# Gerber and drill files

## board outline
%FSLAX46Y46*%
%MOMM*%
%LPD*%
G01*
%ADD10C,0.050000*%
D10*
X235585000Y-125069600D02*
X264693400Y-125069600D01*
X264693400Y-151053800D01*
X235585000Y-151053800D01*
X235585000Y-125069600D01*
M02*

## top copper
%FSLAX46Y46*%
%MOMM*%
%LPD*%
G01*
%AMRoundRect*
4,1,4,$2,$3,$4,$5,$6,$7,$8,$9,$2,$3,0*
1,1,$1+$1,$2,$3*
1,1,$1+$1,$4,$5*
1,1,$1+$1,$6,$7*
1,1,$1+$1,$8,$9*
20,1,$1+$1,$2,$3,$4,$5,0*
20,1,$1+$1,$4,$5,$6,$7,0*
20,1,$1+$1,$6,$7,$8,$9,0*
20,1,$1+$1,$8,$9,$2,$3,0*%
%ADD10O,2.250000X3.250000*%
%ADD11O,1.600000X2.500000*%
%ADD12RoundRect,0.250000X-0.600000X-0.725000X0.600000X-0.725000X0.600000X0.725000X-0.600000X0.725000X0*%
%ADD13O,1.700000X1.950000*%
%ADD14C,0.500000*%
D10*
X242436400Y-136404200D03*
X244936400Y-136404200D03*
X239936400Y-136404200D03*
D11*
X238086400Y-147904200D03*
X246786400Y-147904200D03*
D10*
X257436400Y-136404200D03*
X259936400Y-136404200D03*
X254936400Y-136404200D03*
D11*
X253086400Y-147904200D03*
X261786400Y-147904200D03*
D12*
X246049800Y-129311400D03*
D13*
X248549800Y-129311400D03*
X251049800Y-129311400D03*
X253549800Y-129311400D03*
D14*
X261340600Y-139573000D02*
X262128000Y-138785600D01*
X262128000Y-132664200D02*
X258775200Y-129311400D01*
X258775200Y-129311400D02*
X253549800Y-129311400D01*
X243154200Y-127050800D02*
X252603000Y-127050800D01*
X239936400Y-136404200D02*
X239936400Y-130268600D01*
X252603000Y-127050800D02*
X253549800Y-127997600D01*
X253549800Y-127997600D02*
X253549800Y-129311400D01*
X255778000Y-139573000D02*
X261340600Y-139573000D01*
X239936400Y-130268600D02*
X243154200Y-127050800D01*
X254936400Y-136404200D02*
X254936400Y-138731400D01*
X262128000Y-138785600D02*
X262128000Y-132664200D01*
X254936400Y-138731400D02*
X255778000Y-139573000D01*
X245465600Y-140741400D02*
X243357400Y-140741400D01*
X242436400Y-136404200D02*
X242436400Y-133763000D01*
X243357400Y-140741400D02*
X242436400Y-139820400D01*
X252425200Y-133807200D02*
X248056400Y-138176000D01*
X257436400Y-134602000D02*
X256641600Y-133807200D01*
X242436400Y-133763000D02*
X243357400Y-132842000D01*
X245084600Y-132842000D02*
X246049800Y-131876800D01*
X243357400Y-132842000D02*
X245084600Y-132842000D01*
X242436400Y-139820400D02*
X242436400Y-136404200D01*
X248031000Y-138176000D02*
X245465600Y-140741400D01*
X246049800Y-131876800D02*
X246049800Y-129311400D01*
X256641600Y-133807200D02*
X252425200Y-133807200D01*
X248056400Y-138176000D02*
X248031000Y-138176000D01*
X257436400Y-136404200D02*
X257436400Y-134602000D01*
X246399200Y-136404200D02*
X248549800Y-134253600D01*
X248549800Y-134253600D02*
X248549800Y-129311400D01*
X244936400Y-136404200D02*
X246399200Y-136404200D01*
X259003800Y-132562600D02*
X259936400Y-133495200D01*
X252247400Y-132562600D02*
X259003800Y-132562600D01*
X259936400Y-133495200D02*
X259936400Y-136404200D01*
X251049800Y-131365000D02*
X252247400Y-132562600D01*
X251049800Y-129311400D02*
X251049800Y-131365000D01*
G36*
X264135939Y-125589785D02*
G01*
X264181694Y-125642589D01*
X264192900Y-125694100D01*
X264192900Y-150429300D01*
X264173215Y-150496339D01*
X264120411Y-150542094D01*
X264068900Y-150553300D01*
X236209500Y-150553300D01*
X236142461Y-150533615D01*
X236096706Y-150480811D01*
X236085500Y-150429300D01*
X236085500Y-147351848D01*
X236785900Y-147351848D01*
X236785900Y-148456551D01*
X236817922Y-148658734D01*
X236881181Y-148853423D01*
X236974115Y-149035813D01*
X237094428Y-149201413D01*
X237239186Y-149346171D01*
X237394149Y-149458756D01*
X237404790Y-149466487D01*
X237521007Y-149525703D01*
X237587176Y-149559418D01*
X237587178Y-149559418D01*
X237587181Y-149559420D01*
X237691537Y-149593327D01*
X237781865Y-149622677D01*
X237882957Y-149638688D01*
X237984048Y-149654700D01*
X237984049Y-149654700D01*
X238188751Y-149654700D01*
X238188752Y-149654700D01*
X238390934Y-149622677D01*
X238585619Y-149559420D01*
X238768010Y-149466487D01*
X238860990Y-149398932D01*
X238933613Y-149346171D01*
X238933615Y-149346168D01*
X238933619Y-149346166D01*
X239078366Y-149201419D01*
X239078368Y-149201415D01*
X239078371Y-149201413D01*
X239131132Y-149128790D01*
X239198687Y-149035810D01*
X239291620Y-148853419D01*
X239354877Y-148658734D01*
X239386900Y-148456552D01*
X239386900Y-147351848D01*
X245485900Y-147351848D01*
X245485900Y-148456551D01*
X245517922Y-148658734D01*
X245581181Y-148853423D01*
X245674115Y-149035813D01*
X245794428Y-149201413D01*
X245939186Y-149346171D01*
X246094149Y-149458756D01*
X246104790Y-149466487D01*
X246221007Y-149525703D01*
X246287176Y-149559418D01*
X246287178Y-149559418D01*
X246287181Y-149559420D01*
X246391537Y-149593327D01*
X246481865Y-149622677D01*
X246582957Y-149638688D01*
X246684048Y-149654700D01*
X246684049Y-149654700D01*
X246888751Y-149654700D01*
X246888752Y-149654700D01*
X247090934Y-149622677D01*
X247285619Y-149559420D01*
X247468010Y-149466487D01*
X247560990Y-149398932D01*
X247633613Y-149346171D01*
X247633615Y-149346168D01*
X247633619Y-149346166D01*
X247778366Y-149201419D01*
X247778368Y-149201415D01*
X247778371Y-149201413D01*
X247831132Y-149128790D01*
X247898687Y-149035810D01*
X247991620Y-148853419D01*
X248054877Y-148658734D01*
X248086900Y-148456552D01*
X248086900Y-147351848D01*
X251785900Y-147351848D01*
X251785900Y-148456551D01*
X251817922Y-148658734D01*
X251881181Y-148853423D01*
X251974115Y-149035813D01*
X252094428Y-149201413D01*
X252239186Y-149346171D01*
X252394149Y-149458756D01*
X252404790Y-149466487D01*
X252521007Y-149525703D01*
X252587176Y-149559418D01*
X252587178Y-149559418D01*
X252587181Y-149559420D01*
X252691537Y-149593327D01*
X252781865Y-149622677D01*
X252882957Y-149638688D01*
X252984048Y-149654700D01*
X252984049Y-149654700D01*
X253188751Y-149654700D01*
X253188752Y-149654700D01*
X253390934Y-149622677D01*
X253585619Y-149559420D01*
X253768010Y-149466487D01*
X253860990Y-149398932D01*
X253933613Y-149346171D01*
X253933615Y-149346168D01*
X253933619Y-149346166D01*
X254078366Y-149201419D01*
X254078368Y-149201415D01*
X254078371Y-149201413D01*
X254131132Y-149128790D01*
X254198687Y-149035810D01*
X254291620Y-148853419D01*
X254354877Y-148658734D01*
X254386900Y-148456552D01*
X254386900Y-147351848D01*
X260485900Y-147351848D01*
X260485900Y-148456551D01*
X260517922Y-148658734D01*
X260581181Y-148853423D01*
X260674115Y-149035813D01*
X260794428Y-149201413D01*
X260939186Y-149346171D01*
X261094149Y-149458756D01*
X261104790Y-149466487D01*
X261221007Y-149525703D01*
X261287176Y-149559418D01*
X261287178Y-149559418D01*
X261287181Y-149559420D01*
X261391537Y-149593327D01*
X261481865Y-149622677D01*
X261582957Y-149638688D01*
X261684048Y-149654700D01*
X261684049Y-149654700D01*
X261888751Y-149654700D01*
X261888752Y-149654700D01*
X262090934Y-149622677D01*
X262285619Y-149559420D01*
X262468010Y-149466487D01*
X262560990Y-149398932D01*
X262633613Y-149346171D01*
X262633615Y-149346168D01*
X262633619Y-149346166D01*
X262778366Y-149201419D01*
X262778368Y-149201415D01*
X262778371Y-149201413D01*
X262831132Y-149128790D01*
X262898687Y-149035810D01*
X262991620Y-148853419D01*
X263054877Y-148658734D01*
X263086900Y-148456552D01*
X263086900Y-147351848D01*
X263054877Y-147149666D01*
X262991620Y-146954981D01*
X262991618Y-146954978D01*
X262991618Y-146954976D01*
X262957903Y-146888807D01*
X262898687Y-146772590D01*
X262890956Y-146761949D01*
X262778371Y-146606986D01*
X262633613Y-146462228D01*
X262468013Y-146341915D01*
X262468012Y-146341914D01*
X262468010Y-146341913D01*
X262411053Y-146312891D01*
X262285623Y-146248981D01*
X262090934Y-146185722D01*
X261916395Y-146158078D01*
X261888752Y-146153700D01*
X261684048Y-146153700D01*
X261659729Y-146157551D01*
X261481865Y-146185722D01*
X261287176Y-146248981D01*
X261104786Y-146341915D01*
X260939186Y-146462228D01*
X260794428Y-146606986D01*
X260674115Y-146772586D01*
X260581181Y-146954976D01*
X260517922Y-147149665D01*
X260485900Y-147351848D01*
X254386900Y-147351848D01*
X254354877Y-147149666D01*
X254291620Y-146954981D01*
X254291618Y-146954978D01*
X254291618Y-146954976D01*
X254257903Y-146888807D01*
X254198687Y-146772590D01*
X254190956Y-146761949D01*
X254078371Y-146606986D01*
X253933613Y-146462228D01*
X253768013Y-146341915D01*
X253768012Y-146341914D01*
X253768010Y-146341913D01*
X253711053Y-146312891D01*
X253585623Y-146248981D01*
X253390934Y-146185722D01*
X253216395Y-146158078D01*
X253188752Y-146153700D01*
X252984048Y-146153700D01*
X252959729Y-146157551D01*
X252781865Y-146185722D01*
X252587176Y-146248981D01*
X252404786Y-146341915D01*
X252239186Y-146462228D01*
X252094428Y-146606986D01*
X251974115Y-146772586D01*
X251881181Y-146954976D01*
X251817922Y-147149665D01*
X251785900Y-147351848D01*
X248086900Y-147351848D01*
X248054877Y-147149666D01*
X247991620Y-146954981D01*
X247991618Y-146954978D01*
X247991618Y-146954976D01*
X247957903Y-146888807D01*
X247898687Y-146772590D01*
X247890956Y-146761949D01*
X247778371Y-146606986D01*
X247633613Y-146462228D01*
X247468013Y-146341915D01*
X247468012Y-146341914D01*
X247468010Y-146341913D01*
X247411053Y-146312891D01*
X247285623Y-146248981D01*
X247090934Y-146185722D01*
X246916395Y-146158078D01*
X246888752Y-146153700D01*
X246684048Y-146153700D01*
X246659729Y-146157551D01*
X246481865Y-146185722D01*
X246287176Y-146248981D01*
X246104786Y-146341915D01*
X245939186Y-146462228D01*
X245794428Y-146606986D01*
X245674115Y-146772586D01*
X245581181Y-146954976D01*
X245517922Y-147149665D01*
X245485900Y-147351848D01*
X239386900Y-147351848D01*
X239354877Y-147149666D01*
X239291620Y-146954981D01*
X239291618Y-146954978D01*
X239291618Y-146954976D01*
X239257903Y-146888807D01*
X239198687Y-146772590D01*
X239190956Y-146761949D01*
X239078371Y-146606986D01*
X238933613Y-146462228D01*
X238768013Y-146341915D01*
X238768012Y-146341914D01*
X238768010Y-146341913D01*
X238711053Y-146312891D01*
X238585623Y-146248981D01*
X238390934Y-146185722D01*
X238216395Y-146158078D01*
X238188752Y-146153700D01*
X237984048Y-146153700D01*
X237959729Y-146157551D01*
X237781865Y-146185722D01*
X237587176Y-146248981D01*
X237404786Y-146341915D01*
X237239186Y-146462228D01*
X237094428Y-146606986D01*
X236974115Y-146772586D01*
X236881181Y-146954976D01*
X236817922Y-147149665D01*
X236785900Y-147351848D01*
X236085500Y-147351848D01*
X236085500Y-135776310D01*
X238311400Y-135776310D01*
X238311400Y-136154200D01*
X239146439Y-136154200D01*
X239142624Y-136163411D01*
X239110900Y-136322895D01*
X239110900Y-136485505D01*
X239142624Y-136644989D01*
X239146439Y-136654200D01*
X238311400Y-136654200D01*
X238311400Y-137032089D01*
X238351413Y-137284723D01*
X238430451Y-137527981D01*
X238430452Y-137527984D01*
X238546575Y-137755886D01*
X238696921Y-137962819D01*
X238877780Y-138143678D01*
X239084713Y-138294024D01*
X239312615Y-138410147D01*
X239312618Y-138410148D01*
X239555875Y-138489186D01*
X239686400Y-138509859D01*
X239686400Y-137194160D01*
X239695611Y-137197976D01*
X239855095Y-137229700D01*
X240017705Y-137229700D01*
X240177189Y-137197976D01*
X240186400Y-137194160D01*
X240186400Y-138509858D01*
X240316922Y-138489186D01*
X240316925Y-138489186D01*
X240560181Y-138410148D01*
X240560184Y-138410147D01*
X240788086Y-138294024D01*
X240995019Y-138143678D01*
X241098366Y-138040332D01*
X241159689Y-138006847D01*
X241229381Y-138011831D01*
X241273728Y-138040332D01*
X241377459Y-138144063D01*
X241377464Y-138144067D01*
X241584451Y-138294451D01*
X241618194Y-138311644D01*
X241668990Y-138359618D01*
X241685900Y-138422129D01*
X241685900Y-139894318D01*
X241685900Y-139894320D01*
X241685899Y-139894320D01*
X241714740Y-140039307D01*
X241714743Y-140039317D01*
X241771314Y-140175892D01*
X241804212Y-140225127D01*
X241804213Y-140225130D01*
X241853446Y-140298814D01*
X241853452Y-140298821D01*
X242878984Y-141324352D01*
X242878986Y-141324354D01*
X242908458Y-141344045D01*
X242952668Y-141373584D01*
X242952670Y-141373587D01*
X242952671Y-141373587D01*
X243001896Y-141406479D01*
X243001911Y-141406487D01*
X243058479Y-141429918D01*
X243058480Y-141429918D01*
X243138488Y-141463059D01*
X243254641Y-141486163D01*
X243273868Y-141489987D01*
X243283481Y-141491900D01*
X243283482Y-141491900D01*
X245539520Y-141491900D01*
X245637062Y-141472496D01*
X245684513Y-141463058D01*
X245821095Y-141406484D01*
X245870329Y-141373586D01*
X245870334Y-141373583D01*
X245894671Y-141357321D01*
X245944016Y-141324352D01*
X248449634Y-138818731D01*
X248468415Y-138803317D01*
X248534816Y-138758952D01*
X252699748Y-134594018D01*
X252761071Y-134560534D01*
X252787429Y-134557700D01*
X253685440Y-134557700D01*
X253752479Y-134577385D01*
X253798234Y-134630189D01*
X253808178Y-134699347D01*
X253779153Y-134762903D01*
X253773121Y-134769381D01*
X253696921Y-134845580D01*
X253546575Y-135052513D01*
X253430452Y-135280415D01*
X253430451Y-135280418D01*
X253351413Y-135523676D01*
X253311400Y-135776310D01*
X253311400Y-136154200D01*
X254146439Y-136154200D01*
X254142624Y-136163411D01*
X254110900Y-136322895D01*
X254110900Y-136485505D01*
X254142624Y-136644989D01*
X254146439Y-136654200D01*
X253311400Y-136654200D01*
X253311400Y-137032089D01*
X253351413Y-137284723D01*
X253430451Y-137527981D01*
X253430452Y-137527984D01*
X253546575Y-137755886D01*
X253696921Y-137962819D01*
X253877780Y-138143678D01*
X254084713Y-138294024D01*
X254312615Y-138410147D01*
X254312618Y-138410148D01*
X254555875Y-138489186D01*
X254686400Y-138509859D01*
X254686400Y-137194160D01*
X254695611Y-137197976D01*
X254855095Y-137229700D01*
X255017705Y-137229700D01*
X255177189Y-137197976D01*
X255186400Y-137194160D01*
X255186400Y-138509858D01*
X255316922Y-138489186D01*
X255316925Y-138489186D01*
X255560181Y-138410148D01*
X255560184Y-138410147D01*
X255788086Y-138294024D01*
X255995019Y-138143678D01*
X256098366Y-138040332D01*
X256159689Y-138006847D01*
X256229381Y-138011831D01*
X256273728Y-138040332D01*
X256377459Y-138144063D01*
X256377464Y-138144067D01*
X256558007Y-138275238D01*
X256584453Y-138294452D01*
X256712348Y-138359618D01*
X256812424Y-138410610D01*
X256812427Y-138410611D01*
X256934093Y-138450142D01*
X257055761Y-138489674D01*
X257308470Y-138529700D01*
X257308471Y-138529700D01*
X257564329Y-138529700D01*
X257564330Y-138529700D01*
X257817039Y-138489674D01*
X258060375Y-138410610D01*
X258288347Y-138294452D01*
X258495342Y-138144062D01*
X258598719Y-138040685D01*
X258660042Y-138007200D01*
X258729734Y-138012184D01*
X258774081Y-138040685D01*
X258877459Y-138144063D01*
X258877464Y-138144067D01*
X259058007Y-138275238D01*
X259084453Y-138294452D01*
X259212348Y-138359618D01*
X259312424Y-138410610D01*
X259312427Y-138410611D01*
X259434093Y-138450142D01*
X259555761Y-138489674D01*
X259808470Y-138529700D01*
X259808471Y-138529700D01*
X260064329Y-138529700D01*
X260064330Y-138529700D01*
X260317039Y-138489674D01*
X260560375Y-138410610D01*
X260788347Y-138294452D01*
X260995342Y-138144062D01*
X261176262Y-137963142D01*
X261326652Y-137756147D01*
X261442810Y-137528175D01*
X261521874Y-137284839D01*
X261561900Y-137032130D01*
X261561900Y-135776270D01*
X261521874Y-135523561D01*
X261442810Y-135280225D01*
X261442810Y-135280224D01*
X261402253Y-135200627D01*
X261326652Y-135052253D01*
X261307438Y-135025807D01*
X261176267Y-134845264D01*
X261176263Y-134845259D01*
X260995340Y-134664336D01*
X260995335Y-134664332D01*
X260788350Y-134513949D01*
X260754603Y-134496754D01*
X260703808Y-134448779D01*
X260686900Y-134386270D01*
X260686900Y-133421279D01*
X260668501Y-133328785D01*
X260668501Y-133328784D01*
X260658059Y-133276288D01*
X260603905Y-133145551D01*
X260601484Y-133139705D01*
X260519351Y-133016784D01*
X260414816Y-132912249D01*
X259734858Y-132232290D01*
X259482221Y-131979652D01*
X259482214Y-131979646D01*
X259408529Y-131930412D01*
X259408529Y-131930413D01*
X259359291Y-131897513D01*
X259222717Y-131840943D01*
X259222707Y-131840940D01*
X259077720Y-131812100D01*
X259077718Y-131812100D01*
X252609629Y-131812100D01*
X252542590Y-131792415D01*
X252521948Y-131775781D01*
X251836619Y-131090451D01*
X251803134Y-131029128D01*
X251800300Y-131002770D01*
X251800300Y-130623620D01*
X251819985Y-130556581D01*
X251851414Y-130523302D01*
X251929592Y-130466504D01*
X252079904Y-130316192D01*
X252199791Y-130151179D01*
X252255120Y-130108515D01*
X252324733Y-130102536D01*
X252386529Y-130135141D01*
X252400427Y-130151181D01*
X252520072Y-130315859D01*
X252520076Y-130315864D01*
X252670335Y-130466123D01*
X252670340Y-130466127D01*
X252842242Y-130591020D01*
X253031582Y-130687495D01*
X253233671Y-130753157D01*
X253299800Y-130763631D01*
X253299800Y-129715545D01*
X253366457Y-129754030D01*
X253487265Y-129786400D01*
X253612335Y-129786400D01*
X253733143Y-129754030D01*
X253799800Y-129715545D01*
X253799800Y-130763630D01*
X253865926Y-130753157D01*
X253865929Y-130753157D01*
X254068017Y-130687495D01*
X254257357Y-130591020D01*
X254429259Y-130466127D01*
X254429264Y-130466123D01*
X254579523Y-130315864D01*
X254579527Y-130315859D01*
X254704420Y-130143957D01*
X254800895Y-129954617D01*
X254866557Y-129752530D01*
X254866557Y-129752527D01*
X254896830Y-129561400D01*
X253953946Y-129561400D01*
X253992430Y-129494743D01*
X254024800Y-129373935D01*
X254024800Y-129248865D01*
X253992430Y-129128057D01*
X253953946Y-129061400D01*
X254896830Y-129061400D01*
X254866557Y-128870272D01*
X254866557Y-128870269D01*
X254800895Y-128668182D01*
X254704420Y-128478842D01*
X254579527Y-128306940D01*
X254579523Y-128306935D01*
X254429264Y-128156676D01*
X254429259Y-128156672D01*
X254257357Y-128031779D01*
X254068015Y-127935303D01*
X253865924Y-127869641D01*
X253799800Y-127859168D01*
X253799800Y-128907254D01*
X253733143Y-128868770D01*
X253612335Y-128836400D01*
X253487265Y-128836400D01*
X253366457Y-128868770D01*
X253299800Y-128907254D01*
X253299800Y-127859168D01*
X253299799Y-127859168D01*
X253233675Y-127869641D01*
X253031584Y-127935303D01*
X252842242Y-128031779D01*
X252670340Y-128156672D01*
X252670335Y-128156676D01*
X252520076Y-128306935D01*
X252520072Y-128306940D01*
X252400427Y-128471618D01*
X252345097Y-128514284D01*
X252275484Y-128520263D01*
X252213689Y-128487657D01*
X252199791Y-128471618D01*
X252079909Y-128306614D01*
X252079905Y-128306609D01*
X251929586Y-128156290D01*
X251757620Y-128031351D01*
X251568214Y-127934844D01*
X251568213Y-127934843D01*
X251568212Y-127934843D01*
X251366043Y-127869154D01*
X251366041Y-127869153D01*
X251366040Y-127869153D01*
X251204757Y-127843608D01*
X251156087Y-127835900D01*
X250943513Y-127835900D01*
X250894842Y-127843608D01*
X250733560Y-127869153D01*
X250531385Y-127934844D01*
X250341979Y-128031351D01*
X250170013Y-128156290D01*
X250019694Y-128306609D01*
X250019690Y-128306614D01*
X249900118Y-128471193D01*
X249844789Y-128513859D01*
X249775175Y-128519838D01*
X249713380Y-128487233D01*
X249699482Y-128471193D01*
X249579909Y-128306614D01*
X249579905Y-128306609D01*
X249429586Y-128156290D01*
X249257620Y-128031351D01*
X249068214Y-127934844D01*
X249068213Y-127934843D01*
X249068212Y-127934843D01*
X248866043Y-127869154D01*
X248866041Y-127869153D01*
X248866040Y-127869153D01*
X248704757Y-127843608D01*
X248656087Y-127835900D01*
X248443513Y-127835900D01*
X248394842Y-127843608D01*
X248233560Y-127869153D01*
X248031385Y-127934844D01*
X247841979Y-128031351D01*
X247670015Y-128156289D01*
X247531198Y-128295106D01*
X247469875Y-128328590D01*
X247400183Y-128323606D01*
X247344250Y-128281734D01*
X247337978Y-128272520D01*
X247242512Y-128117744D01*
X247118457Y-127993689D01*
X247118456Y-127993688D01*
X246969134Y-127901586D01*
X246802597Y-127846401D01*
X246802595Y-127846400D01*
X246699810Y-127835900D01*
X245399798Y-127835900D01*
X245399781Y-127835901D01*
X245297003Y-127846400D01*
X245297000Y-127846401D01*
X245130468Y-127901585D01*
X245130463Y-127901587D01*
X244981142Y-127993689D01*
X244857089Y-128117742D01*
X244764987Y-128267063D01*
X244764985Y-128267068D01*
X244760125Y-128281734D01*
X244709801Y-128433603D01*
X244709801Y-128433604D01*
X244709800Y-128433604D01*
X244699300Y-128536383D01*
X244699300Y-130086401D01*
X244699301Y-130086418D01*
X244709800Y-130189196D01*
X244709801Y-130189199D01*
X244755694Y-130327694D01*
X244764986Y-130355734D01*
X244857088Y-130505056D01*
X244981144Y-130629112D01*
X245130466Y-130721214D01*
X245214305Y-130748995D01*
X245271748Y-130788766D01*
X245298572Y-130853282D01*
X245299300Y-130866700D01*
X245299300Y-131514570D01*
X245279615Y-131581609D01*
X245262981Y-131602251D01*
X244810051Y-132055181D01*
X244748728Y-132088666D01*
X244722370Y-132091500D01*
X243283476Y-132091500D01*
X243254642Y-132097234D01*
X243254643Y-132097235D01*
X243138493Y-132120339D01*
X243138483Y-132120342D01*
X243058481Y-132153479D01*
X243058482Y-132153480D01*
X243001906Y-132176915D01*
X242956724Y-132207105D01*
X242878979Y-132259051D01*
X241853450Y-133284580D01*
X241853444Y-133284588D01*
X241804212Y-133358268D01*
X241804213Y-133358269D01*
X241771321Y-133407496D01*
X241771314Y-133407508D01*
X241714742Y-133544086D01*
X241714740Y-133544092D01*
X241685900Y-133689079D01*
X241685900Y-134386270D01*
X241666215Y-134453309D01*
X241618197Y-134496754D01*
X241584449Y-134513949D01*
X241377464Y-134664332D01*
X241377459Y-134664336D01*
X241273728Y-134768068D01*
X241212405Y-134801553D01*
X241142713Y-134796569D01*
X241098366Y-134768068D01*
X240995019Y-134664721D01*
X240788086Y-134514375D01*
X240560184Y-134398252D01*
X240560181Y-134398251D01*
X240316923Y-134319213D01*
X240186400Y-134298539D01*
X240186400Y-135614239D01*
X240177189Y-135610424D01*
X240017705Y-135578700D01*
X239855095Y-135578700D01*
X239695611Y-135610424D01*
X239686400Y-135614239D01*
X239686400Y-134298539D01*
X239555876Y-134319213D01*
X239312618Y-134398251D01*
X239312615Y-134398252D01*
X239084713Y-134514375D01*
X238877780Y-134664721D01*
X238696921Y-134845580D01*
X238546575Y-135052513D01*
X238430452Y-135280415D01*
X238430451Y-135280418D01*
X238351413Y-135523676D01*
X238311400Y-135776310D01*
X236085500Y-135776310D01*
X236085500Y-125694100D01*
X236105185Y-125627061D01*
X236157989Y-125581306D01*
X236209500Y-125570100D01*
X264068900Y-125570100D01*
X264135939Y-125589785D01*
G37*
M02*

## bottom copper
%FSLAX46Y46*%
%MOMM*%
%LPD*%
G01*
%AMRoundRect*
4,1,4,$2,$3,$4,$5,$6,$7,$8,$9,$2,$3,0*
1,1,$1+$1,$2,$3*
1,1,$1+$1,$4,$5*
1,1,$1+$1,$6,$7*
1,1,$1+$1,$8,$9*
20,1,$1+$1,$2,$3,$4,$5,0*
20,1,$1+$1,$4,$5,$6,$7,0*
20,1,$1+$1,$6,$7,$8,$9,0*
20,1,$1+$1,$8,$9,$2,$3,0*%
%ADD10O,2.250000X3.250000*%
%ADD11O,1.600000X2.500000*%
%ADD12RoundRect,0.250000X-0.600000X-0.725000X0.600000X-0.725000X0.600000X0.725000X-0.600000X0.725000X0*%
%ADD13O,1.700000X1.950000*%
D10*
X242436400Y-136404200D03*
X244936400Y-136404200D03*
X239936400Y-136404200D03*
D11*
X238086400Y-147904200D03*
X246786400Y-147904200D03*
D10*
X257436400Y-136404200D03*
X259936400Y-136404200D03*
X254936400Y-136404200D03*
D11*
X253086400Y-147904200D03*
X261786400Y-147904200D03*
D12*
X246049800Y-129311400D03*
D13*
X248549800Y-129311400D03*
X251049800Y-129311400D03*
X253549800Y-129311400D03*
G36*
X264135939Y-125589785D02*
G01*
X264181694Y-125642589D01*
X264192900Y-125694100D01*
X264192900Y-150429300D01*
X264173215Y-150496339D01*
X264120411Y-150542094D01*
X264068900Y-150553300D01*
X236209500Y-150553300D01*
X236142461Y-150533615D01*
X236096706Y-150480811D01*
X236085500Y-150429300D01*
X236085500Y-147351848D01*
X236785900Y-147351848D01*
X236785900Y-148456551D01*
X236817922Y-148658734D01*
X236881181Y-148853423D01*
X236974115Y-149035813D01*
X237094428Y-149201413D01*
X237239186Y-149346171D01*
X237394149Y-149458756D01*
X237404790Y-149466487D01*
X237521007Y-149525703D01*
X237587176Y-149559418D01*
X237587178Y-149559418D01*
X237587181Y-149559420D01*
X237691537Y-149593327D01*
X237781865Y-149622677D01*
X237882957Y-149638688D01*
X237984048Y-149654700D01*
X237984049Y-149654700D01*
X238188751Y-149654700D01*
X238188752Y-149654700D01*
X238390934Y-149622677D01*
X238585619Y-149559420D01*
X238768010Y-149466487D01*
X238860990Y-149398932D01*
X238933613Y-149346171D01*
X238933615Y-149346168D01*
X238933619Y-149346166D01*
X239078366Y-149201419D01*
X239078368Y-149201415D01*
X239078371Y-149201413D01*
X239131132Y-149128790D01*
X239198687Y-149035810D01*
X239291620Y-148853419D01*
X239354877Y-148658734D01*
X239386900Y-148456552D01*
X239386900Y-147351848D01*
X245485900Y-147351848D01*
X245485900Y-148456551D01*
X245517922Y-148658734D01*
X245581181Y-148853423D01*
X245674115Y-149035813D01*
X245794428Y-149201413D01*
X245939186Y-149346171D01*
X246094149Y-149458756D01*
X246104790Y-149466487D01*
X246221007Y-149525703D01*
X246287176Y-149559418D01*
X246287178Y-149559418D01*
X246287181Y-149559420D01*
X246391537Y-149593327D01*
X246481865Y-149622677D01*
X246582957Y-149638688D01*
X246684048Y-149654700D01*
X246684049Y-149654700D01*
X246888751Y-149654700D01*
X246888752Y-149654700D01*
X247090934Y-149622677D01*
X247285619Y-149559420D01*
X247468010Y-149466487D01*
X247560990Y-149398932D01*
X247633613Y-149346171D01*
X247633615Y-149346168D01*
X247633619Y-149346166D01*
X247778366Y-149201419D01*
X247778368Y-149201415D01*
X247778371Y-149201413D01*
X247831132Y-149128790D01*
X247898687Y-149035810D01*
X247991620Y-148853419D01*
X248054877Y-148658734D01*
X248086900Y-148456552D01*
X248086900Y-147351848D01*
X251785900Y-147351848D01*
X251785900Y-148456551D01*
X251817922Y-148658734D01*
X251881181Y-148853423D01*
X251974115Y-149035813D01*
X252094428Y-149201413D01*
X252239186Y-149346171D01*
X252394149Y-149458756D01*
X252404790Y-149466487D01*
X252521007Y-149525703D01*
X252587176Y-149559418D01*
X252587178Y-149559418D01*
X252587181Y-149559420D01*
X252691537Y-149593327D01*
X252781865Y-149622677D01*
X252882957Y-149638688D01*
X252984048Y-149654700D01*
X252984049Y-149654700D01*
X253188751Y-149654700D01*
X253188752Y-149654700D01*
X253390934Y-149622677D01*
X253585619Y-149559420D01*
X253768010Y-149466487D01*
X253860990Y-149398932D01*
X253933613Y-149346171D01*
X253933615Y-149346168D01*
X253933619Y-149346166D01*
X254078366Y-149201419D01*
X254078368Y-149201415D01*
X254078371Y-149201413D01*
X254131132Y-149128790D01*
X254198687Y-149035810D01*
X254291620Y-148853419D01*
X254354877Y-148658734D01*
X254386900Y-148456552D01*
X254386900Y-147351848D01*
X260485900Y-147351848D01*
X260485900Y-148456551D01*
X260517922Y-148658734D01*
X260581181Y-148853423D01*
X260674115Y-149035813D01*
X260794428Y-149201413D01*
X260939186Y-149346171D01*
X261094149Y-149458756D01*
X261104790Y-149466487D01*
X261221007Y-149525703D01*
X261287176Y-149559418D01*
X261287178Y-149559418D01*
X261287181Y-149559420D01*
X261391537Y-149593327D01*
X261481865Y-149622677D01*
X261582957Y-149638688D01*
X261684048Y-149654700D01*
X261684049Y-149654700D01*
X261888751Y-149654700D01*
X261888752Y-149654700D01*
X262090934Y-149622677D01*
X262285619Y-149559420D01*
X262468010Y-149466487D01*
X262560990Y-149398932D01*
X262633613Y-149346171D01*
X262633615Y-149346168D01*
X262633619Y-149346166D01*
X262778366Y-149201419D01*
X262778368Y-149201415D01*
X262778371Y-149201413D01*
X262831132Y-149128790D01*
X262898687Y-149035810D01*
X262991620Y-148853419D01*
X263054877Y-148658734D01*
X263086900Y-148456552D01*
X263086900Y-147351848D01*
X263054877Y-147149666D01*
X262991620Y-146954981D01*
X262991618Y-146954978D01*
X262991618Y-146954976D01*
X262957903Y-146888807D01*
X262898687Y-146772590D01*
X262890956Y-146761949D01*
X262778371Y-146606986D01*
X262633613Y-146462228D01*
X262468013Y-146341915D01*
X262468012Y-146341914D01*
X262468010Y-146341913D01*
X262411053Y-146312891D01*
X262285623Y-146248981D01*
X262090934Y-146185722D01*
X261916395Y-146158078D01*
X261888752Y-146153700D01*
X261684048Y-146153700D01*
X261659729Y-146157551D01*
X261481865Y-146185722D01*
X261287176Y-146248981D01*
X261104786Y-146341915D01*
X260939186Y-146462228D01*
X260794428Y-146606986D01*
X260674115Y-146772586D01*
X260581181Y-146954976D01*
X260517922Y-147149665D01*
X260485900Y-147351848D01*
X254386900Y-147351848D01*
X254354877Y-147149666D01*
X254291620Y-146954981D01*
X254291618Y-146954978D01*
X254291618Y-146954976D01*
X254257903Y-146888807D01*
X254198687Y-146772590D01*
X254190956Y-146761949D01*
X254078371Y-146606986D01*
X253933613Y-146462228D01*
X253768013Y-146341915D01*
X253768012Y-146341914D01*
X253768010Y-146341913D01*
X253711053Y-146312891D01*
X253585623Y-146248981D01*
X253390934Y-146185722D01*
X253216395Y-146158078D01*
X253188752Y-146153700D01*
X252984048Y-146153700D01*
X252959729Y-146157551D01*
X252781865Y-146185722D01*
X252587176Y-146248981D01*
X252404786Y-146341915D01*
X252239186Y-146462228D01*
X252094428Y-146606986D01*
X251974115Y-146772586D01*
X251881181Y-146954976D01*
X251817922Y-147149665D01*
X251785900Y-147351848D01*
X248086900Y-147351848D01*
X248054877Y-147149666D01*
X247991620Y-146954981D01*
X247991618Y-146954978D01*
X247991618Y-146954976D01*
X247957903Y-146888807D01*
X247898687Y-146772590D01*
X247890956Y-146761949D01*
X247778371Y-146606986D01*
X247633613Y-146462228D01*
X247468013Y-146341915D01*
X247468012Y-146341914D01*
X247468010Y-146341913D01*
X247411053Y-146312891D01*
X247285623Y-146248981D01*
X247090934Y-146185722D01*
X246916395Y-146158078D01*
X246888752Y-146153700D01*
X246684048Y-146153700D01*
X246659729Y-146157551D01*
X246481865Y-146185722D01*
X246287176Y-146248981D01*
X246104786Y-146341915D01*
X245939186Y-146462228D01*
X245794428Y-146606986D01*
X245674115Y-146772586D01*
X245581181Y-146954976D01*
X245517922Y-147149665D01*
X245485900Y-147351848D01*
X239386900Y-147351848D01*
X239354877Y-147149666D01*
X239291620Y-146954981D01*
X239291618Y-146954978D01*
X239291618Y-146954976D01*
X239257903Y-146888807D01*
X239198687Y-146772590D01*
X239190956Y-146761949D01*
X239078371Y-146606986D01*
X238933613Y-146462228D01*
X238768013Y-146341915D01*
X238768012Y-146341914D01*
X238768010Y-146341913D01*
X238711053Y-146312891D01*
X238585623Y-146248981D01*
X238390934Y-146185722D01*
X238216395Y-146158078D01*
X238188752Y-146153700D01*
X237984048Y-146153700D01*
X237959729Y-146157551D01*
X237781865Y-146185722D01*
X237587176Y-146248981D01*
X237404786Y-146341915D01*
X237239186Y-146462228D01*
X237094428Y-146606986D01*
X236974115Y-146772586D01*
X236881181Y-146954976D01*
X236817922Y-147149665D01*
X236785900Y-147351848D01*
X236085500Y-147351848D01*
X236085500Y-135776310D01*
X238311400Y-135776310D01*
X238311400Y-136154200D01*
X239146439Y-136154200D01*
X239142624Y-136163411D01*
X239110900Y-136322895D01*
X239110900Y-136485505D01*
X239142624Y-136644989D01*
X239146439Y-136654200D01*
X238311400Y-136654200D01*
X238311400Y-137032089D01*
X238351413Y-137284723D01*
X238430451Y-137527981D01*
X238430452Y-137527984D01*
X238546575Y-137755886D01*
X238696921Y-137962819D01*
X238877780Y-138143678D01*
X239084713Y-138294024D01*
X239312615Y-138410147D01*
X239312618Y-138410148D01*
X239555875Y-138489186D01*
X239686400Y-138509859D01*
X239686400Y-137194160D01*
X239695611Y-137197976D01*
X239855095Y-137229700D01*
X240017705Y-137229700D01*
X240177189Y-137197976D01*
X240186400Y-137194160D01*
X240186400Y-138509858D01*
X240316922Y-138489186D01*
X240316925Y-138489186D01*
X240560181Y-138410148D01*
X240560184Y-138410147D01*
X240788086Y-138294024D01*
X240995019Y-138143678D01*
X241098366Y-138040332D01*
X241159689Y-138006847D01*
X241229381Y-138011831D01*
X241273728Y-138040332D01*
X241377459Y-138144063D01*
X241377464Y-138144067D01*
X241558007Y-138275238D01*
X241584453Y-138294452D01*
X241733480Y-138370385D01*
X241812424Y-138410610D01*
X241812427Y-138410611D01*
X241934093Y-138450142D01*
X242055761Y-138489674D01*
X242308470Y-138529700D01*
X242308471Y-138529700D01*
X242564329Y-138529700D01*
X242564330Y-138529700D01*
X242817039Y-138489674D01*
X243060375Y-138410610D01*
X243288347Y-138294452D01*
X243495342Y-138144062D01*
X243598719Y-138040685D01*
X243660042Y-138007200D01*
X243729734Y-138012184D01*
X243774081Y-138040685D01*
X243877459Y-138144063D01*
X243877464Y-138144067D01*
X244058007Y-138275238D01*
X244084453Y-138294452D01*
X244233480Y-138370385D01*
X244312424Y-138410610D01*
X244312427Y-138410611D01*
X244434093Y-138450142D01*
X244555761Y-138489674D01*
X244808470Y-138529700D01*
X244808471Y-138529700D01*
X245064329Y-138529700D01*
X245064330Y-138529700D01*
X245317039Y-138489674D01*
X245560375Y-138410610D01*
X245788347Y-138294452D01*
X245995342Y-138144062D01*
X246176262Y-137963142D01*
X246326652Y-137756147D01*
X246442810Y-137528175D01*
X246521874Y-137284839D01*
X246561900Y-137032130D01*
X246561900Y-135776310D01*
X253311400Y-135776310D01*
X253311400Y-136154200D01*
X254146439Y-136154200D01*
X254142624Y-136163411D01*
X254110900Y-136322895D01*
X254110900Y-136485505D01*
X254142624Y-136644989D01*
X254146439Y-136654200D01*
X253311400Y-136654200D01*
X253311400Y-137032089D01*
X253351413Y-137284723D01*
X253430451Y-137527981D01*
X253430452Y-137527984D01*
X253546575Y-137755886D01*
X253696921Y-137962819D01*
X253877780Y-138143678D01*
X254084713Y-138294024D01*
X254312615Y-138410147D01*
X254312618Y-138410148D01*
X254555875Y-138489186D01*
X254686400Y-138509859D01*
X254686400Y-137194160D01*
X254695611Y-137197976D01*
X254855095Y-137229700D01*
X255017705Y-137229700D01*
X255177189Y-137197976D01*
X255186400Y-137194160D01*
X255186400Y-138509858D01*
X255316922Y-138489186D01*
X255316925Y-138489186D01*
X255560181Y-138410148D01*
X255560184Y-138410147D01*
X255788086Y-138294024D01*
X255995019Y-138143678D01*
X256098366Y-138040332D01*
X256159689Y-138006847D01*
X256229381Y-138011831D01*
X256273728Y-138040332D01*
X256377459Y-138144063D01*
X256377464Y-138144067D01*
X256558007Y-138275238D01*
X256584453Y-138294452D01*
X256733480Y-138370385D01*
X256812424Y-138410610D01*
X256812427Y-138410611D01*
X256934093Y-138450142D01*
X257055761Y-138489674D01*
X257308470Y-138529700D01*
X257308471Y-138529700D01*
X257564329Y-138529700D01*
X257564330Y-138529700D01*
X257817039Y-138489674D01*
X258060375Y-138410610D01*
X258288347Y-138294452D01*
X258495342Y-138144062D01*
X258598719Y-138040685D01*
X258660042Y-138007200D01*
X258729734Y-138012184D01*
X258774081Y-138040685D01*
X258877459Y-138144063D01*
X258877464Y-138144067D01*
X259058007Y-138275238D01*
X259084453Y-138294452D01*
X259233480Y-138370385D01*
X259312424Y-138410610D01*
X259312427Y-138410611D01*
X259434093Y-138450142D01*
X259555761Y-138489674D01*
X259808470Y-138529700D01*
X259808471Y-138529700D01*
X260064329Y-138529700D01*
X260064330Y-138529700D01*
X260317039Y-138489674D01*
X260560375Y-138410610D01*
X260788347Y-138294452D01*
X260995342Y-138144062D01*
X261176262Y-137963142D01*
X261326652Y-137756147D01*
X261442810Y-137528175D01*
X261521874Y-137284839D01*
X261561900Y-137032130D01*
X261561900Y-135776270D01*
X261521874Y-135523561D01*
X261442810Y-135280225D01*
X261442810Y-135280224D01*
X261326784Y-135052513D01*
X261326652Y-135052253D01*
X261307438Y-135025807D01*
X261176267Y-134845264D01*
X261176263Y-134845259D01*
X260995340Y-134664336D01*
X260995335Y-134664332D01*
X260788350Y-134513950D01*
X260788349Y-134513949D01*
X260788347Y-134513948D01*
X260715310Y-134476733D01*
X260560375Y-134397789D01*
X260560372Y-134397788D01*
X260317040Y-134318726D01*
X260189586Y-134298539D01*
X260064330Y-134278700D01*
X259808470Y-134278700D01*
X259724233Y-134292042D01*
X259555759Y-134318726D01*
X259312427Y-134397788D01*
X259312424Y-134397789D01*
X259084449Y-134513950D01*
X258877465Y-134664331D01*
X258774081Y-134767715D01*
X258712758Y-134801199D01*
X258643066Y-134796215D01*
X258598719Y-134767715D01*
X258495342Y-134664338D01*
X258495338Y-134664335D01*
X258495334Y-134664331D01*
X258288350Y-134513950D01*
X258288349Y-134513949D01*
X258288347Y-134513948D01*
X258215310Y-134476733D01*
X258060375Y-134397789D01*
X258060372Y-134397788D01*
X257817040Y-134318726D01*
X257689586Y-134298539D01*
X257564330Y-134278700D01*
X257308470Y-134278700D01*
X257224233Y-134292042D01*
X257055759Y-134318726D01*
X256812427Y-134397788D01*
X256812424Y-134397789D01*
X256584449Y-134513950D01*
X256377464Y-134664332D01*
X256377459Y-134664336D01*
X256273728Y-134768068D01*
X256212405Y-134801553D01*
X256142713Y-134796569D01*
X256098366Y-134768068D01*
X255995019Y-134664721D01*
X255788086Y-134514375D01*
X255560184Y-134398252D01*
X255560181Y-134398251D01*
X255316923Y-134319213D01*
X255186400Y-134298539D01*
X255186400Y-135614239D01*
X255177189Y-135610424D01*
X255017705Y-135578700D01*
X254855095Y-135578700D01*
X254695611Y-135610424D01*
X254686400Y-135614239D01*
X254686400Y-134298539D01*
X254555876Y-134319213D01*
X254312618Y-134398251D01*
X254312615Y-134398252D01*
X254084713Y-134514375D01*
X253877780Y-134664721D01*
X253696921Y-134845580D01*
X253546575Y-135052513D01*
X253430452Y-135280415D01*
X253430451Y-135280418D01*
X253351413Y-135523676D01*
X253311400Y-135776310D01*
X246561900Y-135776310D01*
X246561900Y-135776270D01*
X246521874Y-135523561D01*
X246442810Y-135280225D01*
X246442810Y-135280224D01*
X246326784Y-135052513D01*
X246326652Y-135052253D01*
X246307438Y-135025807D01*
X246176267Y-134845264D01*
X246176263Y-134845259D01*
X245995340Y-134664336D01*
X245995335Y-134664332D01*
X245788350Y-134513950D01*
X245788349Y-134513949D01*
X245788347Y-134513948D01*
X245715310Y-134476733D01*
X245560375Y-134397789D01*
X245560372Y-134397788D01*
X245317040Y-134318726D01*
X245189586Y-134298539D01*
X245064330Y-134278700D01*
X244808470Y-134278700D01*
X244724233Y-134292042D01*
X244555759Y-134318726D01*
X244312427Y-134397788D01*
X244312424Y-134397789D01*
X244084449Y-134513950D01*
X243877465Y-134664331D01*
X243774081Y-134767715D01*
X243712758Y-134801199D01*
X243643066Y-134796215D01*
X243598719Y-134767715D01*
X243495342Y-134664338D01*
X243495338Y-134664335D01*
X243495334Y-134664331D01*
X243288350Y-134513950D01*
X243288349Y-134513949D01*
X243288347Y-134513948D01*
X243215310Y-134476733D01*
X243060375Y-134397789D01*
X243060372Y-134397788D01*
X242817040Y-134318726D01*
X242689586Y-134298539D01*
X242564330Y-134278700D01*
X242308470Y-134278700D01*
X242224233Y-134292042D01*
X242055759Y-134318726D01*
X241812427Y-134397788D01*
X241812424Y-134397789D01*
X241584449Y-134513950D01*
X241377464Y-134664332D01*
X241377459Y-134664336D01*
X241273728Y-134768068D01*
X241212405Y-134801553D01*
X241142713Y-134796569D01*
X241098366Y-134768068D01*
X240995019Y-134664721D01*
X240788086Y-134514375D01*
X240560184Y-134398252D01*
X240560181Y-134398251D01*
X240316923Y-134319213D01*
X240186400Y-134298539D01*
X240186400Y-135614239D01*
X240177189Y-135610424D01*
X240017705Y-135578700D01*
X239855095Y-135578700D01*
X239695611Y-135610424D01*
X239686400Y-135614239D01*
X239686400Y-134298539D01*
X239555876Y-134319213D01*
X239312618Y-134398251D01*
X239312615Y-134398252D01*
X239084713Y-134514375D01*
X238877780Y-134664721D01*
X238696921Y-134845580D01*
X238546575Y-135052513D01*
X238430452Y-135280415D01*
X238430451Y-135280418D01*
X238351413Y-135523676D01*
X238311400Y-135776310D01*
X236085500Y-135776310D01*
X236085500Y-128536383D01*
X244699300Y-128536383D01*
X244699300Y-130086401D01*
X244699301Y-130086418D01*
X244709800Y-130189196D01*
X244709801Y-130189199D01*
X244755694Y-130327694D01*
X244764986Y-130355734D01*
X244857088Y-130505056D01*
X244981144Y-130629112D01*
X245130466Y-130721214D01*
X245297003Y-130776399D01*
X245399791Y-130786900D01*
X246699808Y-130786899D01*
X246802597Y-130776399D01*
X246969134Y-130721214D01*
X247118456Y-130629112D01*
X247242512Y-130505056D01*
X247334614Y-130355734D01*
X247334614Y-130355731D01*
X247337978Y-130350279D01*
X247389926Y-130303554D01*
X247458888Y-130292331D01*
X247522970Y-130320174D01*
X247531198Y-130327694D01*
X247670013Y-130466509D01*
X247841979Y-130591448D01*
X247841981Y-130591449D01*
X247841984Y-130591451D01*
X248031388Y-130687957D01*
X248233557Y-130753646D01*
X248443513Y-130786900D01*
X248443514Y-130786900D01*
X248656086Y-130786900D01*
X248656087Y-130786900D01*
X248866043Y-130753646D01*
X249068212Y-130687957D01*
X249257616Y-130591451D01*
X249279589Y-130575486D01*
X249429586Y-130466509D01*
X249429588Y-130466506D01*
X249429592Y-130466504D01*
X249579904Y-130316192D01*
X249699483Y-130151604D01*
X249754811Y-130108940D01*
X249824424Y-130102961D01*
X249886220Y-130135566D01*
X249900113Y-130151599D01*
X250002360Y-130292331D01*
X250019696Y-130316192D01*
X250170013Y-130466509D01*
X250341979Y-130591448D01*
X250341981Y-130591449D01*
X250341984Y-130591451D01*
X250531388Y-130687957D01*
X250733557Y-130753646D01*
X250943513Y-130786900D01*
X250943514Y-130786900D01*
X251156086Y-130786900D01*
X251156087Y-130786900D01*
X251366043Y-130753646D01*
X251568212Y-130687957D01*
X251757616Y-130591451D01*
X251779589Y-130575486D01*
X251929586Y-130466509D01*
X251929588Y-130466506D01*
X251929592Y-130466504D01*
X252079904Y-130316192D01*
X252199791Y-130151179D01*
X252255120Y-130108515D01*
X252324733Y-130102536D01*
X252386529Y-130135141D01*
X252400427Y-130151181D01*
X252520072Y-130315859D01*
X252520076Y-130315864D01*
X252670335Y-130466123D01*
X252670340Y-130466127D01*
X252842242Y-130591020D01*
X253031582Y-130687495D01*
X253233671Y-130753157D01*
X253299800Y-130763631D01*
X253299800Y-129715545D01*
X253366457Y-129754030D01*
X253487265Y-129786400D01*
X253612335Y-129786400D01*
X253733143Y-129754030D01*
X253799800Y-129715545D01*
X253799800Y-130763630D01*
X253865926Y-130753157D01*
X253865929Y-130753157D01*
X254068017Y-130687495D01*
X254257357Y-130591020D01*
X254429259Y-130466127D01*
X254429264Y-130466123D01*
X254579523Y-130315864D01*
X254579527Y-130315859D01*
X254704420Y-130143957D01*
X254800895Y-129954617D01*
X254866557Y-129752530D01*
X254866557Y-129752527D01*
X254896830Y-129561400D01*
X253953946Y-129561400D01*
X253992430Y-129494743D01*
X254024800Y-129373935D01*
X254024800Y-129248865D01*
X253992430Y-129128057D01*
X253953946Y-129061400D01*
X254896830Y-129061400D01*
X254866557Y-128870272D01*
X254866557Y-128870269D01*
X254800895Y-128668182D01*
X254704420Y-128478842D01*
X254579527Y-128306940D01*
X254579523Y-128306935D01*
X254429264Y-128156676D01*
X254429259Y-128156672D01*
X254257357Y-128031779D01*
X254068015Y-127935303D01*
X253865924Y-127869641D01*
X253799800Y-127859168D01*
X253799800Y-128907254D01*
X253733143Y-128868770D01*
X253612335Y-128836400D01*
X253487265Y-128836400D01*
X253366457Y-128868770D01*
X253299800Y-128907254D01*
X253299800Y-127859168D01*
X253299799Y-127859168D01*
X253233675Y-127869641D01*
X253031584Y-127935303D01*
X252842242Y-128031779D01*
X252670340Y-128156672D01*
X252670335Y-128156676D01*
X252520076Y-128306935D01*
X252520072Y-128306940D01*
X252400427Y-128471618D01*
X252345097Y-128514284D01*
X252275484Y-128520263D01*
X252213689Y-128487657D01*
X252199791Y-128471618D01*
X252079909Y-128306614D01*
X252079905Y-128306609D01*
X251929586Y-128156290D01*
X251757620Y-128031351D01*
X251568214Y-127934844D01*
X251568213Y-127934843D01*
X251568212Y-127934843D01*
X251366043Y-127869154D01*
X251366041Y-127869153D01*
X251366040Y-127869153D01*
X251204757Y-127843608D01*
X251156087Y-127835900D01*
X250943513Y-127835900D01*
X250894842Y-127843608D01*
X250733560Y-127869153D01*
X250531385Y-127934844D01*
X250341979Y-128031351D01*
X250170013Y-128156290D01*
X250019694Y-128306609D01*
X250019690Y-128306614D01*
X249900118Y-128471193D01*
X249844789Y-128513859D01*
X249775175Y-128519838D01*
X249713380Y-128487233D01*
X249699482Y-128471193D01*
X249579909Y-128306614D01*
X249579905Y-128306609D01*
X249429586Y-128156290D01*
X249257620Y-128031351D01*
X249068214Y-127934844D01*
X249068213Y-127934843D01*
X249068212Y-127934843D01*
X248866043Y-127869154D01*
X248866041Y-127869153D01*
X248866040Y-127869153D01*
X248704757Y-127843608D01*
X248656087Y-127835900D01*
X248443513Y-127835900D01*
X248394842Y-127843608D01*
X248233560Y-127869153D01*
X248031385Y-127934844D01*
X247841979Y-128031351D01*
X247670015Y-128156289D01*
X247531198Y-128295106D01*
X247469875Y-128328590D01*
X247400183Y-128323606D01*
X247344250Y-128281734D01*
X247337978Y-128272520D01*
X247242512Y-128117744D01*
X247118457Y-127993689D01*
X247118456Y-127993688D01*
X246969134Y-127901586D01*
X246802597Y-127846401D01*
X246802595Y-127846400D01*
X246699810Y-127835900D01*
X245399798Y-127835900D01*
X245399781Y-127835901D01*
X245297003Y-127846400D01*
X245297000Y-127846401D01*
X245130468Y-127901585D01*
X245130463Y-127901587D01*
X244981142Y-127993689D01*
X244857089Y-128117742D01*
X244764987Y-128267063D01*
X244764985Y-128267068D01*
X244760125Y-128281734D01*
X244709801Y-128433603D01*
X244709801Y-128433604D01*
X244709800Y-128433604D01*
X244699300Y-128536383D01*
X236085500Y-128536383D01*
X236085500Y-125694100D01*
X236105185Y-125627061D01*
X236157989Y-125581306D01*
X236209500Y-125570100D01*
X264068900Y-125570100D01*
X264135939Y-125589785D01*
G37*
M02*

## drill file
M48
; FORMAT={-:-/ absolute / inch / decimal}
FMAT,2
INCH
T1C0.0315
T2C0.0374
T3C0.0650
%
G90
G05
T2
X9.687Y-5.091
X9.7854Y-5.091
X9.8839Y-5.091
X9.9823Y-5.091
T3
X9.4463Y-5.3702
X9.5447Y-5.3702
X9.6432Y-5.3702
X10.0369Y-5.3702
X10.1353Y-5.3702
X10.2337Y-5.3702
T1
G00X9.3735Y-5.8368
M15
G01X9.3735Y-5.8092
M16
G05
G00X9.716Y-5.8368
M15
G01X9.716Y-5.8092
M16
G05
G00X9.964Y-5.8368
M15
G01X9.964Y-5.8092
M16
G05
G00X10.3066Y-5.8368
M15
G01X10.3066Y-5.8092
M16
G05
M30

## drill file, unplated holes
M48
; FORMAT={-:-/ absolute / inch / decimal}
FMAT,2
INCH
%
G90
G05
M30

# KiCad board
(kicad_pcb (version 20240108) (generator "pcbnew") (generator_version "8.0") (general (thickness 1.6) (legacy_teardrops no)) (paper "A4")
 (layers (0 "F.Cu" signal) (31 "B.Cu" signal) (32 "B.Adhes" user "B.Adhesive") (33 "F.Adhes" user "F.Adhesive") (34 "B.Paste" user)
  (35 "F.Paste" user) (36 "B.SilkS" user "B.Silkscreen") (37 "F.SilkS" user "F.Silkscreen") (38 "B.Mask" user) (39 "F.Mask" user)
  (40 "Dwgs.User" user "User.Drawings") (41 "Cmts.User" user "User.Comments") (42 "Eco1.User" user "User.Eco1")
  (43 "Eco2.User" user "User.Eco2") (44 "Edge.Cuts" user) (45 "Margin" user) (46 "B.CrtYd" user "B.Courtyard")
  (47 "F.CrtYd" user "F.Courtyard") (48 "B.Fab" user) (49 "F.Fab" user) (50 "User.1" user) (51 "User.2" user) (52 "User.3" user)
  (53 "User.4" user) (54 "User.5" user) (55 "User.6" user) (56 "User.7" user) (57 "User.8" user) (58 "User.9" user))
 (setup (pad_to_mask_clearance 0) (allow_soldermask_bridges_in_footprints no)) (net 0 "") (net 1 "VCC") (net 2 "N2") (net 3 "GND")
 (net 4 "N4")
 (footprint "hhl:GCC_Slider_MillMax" (layer "F.Cu") (at 242.4364 136.4042)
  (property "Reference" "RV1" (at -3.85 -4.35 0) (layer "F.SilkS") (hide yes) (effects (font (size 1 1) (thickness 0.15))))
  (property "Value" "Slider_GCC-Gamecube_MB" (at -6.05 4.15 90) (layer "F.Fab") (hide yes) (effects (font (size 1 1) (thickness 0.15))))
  (pad "1" thru_hole oval (at 0 0 180) (size 2.25 3.25) (drill 1.651) (layers "*.Cu" "*.Mask") (remove_unused_layers no) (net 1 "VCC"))
  (pad "2" thru_hole oval (at 2.5 0 180) (size 2.25 3.25) (drill 1.651) (layers "*.Cu" "*.Mask") (remove_unused_layers no) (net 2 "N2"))
  (pad "3" thru_hole oval (at -2.5 0 180) (size 2.25 3.25) (drill 1.651) (layers "*.Cu" "*.Mask") (remove_unused_layers no) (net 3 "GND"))
  (pad "MP" thru_hole oval (at -4.35 11.5 180) (size 1.6 2.5) (drill oval 0.8 1.5) (layers "*.Cu" "*.Mask") (remove_unused_layers no))
  (pad "MP" thru_hole oval (at 4.35 11.5 180) (size 1.6 2.5) (drill oval 0.8 1.5) (layers "*.Cu" "*.Mask") (remove_unused_layers no)))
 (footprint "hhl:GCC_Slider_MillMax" (layer "F.Cu") (at 257.4364 136.4042)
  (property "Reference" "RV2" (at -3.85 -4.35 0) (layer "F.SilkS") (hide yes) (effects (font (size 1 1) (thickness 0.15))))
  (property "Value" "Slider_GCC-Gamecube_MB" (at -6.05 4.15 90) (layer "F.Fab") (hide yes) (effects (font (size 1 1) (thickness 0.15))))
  (pad "1" thru_hole oval (at 0 0 180) (size 2.25 3.25) (drill 1.651) (layers "*.Cu" "*.Mask") (remove_unused_layers no) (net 1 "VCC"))
  (pad "2" thru_hole oval (at 2.5 0 180) (size 2.25 3.25) (drill 1.651) (layers "*.Cu" "*.Mask") (remove_unused_layers no) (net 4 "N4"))
  (pad "3" thru_hole oval (at -2.5 0 180) (size 2.25 3.25) (drill 1.651) (layers "*.Cu" "*.Mask") (remove_unused_layers no) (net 3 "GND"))
  (pad "MP" thru_hole oval (at -4.35 11.5 180) (size 1.6 2.5) (drill oval 0.8 1.5) (layers "*.Cu" "*.Mask") (remove_unused_layers no))
  (pad "MP" thru_hole oval (at 4.35 11.5 180) (size 1.6 2.5) (drill oval 0.8 1.5) (layers "*.Cu" "*.Mask") (remove_unused_layers no)))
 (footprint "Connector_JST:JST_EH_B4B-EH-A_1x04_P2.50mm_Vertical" (layer "F.Cu") (at 246.0498 129.3114)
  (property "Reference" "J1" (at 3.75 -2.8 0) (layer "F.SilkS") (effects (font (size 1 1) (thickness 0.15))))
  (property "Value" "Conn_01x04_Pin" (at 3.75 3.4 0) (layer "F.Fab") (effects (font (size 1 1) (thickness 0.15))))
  (pad "1" thru_hole roundrect (at 0 0) (size 1.7 1.95) (drill 0.95) (layers "*.Cu" "*.Mask") (remove_unused_layers no)
   (roundrect_rratio 0.147059) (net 1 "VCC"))
  (pad "2" thru_hole oval (at 2.5 0) (size 1.7 1.95) (drill 0.95) (layers "*.Cu" "*.Mask") (remove_unused_layers no) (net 2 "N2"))
  (pad "3" thru_hole oval (at 5 0) (size 1.7 1.95) (drill 0.95) (layers "*.Cu" "*.Mask") (remove_unused_layers no) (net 4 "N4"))
  (pad "4" thru_hole oval (at 7.5 0) (size 1.7 1.95) (drill 0.95) (layers "*.Cu" "*.Mask") (remove_unused_layers no) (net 3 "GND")))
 (gr_rect (start 235.585 125.0696) (end 264.6934 151.0538) (stroke (width 0.05) (type default)) (fill none) (layer "Edge.Cuts"))
 (segment (start 261.3406 139.573) (end 262.128 138.7856) (width 0.5) (layer "F.Cu") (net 3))
 (segment (start 262.128 132.6642) (end 258.7752 129.3114) (width 0.5) (layer "F.Cu") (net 3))
 (segment (start 258.7752 129.3114) (end 253.5498 129.3114) (width 0.5) (layer "F.Cu") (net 3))
 (segment (start 243.1542 127.0508) (end 252.603 127.0508) (width 0.5) (layer "F.Cu") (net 3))
 (segment (start 239.9364 136.4042) (end 239.9364 130.2686) (width 0.5) (layer "F.Cu") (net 3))
 (segment (start 252.603 127.0508) (end 253.5498 127.9976) (width 0.5) (layer "F.Cu") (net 3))
 (segment (start 253.5498 127.9976) (end 253.5498 129.3114) (width 0.5) (layer "F.Cu") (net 3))
 (segment (start 255.778 139.573) (end 261.3406 139.573) (width 0.5) (layer "F.Cu") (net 3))
 (segment (start 239.9364 130.2686) (end 243.1542 127.0508) (width 0.5) (layer "F.Cu") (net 3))
 (segment (start 254.9364 136.4042) (end 254.9364 138.7314) (width 0.5) (layer "F.Cu") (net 3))
 (segment (start 262.128 138.7856) (end 262.128 132.6642) (width 0.5) (layer "F.Cu") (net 3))
 (segment (start 254.9364 138.7314) (end 255.778 139.573) (width 0.5) (layer "F.Cu") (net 3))
 (segment (start 245.4656 140.7414) (end 243.3574 140.7414) (width 0.5) (layer "F.Cu") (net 1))
 (segment (start 242.4364 136.4042) (end 242.4364 133.763) (width 0.5) (layer "F.Cu") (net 1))
 (segment (start 243.3574 140.7414) (end 242.4364 139.8204) (width 0.5) (layer "F.Cu") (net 1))
 (segment (start 252.4252 133.8072) (end 248.0564 138.176) (width 0.5) (layer "F.Cu") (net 1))
 (segment (start 257.4364 134.602) (end 256.6416 133.8072) (width 0.5) (layer "F.Cu") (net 1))
 (segment (start 242.4364 133.763) (end 243.3574 132.842) (width 0.5) (layer "F.Cu") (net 1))
 (segment (start 245.0846 132.842) (end 246.0498 131.8768) (width 0.5) (layer "F.Cu") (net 1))
 (segment (start 243.3574 132.842) (end 245.0846 132.842) (width 0.5) (layer "F.Cu") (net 1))
 (segment (start 242.4364 139.8204) (end 242.4364 136.4042) (width 0.5) (layer "F.Cu") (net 1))
 (segment (start 248.031 138.176) (end 245.4656 140.7414) (width 0.5) (layer "F.Cu") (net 1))
 (segment (start 246.0498 131.8768) (end 246.0498 129.3114) (width 0.5) (layer "F.Cu") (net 1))
 (segment (start 256.6416 133.8072) (end 252.4252 133.8072) (width 0.5) (layer "F.Cu") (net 1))
 (segment (start 248.0564 138.176) (end 248.031 138.176) (width 0.5) (layer "F.Cu") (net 1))
 (segment (start 257.4364 136.4042) (end 257.4364 134.602) (width 0.5) (layer "F.Cu") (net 1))
 (segment (start 246.3992 136.4042) (end 248.5498 134.2536) (width 0.5) (layer "F.Cu") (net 2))
 (segment (start 248.5498 134.2536) (end 248.5498 129.3114) (width 0.5) (layer "F.Cu") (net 2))
 (segment (start 244.9364 136.4042) (end 246.3992 136.4042) (width 0.5) (layer "F.Cu") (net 2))
 (segment (start 259.0038 132.5626) (end 259.9364 133.4952) (width 0.5) (layer "F.Cu") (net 4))
 (segment (start 252.2474 132.5626) (end 259.0038 132.5626) (width 0.5) (layer "F.Cu") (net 4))
 (segment (start 259.9364 133.4952) (end 259.9364 136.4042) (width 0.5) (layer "F.Cu") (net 4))
 (segment (start 251.0498 131.365) (end 252.2474 132.5626) (width 0.5) (layer "F.Cu") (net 4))
 (segment (start 251.0498 129.3114) (end 251.0498 131.365) (width 0.5) (layer "F.Cu") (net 4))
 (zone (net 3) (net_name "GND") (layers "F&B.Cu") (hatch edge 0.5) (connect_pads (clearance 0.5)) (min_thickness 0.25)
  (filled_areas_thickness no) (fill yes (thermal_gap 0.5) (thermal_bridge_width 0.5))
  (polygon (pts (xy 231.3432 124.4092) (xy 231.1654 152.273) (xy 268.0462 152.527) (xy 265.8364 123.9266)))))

